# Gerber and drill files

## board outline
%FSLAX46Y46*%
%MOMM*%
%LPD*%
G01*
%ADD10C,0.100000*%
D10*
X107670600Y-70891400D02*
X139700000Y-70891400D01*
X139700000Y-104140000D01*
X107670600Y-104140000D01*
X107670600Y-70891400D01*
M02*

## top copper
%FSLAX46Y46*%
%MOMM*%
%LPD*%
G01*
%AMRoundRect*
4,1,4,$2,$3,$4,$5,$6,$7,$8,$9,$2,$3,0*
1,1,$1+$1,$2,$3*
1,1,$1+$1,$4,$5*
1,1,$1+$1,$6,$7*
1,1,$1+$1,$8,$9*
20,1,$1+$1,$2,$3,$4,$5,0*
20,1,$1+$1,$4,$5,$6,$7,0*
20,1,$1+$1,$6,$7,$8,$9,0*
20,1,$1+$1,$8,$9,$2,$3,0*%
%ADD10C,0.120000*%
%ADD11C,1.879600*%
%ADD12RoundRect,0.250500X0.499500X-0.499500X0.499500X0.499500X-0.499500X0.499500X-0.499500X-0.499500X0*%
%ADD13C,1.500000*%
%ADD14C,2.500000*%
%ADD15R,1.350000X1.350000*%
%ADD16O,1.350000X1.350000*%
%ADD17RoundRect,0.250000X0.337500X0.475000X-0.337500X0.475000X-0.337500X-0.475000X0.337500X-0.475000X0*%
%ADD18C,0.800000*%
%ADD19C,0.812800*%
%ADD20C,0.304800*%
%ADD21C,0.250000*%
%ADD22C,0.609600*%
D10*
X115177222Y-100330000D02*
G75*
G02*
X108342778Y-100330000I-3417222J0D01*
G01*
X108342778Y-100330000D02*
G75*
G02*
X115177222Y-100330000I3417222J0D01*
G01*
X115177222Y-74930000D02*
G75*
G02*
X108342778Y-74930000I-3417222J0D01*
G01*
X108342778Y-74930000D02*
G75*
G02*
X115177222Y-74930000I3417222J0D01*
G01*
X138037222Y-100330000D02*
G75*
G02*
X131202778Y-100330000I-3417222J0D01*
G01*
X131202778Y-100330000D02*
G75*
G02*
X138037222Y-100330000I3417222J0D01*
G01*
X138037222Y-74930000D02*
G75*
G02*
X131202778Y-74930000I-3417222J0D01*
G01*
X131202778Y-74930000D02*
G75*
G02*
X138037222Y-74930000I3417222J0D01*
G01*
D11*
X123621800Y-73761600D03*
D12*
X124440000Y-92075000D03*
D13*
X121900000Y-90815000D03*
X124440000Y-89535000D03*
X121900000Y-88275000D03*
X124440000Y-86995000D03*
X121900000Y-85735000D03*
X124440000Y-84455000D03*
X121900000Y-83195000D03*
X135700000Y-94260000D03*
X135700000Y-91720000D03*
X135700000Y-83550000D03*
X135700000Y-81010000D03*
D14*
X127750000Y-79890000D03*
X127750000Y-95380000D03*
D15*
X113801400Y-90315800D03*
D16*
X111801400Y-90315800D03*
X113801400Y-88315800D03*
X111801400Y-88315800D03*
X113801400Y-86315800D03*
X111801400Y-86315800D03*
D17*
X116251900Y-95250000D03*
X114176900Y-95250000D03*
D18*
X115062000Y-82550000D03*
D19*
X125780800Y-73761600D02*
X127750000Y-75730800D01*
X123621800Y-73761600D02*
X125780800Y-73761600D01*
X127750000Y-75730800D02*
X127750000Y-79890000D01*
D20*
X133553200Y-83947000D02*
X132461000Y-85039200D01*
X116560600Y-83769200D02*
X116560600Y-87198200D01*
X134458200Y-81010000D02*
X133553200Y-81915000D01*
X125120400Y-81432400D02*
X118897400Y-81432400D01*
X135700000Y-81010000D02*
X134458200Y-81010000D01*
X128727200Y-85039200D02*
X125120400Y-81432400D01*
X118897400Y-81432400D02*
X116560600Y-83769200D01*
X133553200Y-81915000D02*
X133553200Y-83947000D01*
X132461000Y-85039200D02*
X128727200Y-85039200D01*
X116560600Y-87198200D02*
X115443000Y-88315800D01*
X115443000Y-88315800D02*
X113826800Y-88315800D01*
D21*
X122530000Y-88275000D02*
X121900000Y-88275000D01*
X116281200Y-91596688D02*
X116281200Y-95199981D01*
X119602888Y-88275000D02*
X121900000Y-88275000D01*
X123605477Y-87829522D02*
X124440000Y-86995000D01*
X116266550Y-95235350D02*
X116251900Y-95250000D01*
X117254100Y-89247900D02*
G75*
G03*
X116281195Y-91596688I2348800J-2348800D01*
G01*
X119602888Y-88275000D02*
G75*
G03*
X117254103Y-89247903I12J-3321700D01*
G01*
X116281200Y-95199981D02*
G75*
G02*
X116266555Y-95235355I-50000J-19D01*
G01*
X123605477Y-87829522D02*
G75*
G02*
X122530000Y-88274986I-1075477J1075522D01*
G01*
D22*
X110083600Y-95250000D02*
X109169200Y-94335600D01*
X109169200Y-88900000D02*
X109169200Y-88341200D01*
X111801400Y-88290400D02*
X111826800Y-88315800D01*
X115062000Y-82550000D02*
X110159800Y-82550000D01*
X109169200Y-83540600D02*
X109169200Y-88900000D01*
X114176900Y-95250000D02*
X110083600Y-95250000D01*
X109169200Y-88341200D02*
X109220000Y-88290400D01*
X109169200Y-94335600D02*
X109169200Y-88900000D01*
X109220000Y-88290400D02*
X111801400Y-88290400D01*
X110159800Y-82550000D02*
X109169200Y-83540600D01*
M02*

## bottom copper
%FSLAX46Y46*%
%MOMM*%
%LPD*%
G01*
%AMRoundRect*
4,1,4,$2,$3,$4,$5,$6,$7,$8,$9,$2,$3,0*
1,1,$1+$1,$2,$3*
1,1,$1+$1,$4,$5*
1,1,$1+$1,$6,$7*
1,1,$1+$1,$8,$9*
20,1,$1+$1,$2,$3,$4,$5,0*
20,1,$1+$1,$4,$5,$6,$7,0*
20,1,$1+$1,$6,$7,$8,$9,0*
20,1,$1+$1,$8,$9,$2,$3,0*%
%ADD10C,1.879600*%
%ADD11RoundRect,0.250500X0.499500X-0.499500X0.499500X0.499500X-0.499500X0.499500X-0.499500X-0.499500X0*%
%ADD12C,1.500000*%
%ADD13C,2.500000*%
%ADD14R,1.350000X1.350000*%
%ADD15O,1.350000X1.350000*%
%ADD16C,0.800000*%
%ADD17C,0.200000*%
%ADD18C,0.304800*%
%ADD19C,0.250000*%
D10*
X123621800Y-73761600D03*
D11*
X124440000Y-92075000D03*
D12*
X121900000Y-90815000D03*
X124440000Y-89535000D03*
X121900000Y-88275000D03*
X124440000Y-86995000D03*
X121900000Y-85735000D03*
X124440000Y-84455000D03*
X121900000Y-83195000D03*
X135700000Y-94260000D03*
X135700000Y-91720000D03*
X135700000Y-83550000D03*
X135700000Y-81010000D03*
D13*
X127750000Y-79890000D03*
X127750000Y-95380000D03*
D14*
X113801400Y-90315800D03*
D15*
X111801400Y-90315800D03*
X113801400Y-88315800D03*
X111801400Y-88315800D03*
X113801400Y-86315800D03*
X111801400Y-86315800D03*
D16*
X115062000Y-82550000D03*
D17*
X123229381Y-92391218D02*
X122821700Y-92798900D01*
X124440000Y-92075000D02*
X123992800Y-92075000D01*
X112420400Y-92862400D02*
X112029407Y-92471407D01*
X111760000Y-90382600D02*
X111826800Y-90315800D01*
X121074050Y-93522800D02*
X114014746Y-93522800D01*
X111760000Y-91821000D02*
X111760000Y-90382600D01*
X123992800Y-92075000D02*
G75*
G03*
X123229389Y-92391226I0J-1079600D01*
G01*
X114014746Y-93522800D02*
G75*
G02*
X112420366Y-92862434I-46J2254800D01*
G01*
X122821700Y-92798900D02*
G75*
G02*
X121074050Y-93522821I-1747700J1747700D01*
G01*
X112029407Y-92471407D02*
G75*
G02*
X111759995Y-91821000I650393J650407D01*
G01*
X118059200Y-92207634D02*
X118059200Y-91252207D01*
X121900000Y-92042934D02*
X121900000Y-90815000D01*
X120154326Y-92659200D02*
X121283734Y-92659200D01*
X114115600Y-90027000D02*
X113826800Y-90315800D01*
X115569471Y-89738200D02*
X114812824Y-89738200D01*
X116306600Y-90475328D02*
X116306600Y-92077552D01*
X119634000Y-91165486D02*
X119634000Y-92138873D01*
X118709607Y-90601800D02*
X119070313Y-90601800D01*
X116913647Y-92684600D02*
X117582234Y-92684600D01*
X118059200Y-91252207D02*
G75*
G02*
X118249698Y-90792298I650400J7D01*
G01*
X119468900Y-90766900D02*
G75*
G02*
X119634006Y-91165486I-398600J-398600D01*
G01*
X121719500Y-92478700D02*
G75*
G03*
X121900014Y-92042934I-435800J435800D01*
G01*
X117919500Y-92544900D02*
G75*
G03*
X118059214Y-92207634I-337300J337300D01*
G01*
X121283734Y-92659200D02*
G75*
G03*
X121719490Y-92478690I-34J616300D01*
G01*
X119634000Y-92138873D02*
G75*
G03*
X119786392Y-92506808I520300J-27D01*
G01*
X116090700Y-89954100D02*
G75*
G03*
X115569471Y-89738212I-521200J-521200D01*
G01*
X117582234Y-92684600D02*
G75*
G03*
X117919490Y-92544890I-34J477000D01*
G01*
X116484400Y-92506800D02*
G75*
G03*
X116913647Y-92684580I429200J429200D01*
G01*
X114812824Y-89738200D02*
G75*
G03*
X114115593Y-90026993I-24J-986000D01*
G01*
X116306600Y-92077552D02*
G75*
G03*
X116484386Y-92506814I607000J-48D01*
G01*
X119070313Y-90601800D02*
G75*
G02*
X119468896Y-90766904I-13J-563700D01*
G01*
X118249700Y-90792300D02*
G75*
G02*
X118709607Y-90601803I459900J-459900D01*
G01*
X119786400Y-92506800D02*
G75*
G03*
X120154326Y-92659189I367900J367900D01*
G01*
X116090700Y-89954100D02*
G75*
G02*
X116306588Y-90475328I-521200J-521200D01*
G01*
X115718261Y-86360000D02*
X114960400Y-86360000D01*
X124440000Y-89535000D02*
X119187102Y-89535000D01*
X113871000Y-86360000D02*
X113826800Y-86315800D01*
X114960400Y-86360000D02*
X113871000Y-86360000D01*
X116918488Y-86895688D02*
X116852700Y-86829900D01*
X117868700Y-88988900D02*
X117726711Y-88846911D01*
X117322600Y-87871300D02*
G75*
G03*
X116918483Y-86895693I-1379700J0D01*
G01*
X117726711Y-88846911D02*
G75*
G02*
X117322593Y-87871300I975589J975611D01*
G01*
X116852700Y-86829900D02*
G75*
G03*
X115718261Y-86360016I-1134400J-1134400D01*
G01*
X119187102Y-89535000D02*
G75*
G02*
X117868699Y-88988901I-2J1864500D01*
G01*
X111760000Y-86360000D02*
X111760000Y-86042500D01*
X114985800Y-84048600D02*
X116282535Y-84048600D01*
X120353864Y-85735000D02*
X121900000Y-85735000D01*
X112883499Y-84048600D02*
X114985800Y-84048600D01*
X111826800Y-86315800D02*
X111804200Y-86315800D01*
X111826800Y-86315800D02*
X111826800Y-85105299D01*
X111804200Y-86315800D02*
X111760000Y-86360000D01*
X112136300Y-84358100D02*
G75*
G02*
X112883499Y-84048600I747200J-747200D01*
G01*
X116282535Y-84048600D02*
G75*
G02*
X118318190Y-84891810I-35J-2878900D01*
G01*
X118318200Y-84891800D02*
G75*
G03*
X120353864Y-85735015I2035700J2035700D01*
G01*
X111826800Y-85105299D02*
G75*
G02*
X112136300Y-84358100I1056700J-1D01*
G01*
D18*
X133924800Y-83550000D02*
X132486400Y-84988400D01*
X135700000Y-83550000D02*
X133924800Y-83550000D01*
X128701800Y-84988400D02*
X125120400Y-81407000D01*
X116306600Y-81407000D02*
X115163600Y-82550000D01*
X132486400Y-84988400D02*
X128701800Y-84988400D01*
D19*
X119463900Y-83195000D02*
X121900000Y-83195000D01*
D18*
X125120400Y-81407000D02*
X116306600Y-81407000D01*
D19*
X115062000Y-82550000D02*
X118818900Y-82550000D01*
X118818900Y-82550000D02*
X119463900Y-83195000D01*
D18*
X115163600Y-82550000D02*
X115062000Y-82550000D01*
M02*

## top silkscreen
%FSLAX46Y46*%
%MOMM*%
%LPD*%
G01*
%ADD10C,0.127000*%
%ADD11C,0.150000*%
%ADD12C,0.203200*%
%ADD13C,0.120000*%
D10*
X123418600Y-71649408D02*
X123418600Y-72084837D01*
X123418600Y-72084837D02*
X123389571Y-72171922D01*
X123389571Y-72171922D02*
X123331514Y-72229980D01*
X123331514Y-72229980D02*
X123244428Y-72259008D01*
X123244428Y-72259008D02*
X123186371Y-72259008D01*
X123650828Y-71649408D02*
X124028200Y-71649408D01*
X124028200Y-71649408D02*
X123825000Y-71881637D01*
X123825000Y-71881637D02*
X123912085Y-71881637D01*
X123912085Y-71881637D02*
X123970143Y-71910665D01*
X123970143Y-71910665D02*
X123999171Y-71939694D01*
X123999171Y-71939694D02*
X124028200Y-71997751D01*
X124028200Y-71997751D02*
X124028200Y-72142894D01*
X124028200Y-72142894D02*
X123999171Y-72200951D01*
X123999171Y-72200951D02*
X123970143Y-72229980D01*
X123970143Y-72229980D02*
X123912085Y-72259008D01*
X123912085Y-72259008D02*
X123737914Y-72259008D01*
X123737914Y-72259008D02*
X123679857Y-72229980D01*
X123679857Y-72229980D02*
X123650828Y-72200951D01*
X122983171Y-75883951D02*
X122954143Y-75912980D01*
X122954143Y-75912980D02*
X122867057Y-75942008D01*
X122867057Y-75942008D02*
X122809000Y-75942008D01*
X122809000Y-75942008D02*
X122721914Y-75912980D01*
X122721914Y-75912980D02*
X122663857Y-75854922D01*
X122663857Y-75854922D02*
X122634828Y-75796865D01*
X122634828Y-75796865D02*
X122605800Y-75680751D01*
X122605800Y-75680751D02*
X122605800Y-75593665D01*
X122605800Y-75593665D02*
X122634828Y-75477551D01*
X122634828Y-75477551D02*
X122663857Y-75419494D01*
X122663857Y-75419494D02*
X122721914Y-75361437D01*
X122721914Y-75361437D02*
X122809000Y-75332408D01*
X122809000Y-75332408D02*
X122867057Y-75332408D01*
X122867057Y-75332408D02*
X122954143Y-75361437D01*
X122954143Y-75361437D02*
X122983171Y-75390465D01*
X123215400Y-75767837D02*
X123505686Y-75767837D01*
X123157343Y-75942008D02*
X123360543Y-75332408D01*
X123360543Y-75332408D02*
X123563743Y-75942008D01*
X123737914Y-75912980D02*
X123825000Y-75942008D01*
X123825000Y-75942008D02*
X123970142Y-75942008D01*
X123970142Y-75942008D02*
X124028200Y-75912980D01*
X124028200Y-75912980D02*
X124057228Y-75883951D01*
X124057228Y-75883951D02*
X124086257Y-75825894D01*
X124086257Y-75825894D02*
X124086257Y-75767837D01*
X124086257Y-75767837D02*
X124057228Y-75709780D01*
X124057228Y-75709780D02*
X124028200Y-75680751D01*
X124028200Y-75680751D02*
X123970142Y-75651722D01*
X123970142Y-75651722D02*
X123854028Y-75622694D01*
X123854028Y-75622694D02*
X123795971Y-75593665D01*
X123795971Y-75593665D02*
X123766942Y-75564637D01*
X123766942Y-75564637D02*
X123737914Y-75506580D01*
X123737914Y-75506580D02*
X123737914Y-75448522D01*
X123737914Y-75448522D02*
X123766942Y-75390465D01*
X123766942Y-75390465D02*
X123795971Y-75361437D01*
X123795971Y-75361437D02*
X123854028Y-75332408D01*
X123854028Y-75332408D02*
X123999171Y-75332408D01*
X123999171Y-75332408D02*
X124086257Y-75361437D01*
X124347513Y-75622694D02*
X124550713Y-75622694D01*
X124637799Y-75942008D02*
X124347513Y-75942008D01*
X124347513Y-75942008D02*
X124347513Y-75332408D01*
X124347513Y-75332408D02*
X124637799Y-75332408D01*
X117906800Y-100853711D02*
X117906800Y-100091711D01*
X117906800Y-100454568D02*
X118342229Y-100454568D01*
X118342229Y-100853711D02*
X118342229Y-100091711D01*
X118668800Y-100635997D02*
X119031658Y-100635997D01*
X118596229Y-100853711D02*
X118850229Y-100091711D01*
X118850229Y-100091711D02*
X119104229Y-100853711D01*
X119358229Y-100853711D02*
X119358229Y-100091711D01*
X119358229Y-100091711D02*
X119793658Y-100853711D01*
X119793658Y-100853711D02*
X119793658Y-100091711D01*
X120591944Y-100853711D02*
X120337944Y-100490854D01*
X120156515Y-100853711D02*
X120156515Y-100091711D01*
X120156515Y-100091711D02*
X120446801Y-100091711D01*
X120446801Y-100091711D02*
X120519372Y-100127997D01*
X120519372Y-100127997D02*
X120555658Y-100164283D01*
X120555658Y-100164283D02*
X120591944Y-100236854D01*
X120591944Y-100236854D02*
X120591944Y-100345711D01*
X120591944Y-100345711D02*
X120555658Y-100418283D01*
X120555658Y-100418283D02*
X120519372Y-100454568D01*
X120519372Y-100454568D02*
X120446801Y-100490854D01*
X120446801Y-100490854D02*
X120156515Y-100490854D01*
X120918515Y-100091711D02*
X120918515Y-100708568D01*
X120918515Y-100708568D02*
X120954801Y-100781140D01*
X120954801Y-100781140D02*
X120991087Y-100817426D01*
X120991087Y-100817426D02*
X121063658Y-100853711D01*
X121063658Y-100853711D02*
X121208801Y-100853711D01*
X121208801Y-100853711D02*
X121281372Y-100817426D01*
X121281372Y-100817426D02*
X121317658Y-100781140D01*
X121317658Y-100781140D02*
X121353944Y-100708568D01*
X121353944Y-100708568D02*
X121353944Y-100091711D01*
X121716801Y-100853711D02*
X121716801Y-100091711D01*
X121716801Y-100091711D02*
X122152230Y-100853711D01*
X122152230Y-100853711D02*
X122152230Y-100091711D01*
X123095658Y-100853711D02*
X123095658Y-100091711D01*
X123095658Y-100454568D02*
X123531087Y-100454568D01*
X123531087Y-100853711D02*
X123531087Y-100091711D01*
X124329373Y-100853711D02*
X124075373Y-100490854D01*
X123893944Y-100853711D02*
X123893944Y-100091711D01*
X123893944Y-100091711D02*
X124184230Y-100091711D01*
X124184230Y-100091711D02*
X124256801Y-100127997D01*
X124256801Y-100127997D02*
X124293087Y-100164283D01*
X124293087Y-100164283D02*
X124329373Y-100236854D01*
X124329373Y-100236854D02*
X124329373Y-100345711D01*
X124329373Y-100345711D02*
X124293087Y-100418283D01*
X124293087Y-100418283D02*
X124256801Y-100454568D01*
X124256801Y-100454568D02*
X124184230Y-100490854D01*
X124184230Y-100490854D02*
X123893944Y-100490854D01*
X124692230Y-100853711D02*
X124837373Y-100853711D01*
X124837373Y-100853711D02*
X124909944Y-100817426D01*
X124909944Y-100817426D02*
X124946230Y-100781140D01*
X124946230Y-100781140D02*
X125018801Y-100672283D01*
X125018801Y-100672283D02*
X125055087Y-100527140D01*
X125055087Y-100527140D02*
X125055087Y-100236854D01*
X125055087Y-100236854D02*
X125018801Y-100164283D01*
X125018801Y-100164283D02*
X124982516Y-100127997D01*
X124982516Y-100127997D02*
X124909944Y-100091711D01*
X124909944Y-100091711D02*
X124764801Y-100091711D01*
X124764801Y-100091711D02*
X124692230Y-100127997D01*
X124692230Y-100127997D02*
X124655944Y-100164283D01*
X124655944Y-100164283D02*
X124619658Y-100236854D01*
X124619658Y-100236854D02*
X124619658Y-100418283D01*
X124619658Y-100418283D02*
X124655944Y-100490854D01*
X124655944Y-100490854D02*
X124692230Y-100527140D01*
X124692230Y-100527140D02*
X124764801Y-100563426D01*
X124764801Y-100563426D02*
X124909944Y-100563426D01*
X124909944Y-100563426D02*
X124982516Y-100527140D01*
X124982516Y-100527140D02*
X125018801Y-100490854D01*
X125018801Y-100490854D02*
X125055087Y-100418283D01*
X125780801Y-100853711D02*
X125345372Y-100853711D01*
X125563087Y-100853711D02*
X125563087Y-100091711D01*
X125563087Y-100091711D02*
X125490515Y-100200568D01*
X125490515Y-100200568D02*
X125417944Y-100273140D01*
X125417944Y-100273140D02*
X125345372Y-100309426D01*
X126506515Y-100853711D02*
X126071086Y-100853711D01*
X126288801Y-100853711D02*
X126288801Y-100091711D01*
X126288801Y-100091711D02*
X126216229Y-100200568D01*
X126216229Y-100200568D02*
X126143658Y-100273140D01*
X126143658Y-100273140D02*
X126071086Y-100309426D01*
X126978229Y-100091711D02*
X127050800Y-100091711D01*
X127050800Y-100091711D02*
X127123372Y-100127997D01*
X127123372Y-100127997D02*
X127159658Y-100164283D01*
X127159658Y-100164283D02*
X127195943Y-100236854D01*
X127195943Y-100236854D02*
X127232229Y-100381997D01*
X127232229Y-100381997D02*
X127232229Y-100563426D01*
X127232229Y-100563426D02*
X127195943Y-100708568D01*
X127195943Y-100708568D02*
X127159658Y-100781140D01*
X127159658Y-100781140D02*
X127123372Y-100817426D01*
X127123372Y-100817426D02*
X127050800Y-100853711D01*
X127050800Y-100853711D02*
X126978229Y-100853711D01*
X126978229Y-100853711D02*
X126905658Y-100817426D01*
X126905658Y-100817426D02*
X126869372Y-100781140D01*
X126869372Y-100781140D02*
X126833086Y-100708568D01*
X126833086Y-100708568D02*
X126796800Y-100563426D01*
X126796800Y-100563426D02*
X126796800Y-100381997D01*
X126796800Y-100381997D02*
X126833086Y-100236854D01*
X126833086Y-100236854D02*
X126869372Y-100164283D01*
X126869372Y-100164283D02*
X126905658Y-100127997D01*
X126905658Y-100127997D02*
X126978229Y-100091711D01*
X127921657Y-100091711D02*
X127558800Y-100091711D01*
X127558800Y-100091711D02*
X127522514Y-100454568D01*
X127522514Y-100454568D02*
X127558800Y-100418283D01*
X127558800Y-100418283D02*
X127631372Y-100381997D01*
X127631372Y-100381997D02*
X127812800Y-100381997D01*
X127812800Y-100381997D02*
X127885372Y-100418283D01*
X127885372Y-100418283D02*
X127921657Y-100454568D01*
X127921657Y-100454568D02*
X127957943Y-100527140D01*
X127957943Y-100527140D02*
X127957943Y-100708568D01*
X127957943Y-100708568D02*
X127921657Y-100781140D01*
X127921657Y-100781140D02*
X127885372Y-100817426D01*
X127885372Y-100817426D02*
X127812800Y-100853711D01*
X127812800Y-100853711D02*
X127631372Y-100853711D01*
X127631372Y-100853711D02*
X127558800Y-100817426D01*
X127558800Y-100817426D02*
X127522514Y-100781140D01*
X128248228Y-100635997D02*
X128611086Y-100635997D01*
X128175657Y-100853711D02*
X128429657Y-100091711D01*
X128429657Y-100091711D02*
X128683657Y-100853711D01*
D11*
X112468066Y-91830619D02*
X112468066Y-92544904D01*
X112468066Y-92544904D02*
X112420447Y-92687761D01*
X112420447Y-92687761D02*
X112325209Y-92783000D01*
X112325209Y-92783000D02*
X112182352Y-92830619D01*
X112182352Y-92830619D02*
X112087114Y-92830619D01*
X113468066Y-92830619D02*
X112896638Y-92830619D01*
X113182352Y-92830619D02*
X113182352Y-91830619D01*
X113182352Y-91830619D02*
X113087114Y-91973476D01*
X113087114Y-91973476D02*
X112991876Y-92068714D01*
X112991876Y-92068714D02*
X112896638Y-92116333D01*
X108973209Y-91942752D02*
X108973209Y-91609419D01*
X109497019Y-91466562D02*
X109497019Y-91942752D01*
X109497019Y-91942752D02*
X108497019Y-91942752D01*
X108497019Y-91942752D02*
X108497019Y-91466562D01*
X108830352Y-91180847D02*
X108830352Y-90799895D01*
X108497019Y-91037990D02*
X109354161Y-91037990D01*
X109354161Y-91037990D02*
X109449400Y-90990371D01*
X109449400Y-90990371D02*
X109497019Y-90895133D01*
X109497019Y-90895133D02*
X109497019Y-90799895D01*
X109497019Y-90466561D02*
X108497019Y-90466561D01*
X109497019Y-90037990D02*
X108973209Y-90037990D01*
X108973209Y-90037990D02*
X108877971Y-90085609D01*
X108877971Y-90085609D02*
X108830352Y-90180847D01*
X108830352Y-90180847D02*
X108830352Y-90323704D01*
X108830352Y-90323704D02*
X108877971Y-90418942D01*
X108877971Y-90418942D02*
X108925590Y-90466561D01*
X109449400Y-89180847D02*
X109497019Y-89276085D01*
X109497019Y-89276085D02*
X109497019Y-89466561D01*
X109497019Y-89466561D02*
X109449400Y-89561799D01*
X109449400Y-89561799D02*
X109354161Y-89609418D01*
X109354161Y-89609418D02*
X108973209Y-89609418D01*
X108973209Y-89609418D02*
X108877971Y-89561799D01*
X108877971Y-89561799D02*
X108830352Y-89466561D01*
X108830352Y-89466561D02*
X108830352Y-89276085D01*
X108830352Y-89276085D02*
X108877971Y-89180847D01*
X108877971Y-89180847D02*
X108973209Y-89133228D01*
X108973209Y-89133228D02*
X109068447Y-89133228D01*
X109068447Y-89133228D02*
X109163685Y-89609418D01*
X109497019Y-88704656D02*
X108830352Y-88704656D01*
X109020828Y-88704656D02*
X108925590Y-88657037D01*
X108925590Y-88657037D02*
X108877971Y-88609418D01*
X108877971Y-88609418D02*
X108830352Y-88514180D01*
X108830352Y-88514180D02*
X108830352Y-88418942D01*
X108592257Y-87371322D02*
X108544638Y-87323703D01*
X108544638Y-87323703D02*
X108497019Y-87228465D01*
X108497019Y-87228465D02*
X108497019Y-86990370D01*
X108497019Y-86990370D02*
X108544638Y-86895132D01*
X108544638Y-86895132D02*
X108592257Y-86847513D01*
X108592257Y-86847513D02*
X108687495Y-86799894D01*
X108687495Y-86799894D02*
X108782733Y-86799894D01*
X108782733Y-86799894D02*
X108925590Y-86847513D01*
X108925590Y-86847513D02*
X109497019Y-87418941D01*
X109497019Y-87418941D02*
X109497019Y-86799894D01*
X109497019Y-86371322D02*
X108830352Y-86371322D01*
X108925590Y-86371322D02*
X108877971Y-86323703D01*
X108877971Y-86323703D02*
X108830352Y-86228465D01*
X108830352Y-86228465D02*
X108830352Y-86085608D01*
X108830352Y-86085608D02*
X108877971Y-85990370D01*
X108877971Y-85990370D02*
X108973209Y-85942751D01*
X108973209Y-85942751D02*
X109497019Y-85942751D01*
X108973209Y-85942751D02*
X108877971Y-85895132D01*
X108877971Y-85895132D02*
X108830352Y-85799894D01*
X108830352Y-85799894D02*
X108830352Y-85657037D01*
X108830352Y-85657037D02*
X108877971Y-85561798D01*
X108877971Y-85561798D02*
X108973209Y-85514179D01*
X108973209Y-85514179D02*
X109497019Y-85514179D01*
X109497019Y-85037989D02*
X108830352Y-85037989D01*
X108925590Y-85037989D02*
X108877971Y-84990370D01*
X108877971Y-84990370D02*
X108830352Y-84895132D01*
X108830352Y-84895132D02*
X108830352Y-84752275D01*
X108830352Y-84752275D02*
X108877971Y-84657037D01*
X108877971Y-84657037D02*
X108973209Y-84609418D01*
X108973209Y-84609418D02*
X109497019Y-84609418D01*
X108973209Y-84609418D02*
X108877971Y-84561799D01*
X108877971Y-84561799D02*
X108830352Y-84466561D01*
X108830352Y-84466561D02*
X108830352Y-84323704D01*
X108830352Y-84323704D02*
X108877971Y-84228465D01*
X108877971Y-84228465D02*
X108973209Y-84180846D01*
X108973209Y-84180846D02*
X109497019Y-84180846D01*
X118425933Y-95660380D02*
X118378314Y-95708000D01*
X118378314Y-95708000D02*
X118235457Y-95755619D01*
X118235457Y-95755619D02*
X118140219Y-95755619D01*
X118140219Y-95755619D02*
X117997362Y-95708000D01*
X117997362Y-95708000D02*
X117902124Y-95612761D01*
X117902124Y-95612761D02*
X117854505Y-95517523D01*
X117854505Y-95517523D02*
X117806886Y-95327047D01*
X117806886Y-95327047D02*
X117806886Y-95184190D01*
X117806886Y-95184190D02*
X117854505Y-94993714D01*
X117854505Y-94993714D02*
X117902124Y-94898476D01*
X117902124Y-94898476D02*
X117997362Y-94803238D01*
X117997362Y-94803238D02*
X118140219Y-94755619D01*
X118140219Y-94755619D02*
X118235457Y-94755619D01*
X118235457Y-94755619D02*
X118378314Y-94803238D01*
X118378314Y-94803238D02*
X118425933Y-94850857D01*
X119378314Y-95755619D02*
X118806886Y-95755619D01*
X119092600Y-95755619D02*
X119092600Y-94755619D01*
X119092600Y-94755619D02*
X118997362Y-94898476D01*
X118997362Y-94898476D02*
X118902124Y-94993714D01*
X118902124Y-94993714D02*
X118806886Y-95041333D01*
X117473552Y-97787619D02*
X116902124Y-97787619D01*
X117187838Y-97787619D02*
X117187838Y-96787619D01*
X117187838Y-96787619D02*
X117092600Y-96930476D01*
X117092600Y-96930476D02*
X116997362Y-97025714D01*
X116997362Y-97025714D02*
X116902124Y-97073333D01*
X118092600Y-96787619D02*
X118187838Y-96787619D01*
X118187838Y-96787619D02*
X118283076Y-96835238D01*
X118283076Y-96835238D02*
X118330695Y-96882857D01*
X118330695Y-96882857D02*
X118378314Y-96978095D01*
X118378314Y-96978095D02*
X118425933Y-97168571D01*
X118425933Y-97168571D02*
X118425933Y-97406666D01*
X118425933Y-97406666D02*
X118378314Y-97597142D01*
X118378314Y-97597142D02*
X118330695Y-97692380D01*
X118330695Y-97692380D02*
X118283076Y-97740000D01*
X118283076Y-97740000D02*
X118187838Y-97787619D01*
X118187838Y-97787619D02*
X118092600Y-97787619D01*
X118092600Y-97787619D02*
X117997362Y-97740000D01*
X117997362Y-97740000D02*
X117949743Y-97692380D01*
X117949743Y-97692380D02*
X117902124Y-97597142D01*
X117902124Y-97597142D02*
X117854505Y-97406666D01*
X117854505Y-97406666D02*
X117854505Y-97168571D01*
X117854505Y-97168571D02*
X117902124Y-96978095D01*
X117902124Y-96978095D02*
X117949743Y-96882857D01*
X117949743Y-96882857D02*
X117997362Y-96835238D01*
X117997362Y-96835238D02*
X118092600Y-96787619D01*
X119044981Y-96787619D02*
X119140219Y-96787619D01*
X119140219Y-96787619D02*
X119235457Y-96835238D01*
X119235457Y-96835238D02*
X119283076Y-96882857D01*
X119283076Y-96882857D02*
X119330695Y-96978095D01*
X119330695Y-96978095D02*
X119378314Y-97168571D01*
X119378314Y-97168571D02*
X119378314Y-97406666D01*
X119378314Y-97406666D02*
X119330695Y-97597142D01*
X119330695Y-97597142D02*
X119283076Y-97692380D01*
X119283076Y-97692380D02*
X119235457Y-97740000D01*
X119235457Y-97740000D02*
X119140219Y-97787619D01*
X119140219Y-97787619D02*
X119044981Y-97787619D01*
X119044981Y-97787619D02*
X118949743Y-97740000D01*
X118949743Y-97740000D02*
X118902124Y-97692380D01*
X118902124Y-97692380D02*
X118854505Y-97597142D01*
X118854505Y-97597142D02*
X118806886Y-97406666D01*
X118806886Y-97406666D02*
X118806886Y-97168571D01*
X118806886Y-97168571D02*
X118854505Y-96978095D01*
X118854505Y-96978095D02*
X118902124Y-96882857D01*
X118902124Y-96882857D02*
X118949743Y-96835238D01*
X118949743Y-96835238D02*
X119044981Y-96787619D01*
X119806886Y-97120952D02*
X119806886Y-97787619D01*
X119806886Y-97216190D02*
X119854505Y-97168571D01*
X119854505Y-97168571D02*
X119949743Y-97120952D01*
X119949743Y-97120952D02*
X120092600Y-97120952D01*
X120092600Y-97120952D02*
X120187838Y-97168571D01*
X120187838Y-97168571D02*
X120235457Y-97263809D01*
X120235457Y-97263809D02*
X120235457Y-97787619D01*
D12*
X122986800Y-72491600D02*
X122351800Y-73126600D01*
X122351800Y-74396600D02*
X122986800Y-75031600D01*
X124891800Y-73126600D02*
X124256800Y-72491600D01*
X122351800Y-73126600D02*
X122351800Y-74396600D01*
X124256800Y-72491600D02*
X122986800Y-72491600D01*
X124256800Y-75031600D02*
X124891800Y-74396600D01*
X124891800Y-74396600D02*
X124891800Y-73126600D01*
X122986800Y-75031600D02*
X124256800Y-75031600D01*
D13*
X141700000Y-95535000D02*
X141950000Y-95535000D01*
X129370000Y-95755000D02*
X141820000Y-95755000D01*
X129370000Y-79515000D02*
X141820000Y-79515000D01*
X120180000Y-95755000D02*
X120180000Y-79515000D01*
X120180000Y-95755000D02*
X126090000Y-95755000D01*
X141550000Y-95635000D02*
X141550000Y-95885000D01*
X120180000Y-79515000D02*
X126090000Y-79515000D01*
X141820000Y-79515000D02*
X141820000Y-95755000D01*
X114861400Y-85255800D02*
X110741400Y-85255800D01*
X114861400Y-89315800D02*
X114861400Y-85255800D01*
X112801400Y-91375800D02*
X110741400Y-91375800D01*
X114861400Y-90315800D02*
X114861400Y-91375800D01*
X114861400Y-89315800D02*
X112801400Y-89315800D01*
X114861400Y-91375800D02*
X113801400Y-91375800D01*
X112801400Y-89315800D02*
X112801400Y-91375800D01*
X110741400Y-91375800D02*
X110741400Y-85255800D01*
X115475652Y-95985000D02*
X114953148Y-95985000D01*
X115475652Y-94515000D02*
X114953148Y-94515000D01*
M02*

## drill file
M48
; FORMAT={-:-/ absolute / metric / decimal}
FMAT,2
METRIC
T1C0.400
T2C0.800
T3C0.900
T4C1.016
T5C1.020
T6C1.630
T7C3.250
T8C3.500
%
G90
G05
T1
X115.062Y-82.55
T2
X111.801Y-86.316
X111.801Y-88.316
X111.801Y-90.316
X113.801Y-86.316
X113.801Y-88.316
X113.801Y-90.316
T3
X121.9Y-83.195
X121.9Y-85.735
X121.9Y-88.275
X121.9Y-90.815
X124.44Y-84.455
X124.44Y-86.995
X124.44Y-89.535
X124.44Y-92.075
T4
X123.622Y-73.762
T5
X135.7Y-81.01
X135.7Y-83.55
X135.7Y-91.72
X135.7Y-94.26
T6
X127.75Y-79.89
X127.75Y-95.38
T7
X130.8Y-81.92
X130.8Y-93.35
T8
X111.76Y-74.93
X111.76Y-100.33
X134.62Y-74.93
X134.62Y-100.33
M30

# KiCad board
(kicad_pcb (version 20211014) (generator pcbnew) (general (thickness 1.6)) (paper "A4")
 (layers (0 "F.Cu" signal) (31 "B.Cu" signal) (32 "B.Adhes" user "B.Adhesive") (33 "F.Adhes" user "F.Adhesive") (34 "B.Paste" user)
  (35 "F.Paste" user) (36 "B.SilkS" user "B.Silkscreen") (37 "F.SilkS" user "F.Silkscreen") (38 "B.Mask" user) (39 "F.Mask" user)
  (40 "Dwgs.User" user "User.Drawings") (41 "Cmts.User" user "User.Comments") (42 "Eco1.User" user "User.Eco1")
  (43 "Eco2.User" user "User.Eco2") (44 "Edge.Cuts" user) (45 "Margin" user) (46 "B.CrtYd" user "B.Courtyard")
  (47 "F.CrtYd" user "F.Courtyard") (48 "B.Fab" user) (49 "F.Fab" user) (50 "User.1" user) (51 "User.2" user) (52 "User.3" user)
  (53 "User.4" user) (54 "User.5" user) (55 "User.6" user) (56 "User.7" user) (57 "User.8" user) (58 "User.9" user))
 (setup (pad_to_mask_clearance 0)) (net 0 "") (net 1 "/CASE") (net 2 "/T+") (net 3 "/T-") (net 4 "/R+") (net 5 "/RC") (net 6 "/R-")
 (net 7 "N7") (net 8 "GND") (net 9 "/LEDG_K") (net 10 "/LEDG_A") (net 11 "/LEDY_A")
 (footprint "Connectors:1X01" (layer "F.Cu") (at 123.6218 73.7616)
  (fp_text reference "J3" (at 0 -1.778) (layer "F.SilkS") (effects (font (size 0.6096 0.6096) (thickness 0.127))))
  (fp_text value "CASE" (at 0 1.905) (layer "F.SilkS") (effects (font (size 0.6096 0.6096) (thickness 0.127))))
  (fp_line (start -0.635 -1.27) (end -1.27 -0.635) (layer "F.SilkS") (width 0.2032))
  (fp_line (start -1.27 0.635) (end -0.635 1.27) (layer "F.SilkS") (width 0.2032))
  (fp_line (start 1.27 -0.635) (end 0.635 -1.27) (layer "F.SilkS") (width 0.2032))
  (fp_line (start -1.27 -0.635) (end -1.27 0.635) (layer "F.SilkS") (width 0.2032))
  (fp_line (start 0.635 -1.27) (end -0.635 -1.27) (layer "F.SilkS") (width 0.2032))
  (fp_line (start 0.635 1.27) (end 1.27 0.635) (layer "F.SilkS") (width 0.2032))
  (fp_line (start 1.27 0.635) (end 1.27 -0.635) (layer "F.SilkS") (width 0.2032))
  (fp_line (start -0.635 1.27) (end 0.635 1.27) (layer "F.SilkS") (width 0.2032))
  (pad "1" thru_hole circle locked (at 0 0) (size 1.8796 1.8796) (drill 1.016) (layers *.Cu *.Mask) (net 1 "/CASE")
   (solder_mask_margin 0.1016)))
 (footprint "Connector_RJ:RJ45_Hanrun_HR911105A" (layer "F.Cu") (at 124.44 92.075 90)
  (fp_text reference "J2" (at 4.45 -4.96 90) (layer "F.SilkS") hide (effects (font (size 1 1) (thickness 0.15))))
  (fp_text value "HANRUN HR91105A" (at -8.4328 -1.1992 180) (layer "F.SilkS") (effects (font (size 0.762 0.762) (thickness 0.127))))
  (fp_line (start -3.46 17.26) (end -3.46 17.51) (layer "F.SilkS") (width 0.12))
  (fp_line (start -3.68 4.93) (end -3.68 17.38) (layer "F.SilkS") (width 0.12))
  (fp_line (start 12.56 4.93) (end 12.56 17.38) (layer "F.SilkS") (width 0.12))
  (fp_line (start -3.68 -4.26) (end 12.56 -4.26) (layer "F.SilkS") (width 0.12))
  (fp_line (start -3.68 -4.26) (end -3.68 1.65) (layer "F.SilkS") (width 0.12))
  (fp_line (start -3.56 17.11) (end -3.81 17.11) (layer "F.SilkS") (width 0.12))
  (fp_line (start 12.56 -4.26) (end 12.56 1.65) (layer "F.SilkS") (width 0.12))
  (fp_line (start 12.56 17.38) (end -3.68 17.38) (layer "F.SilkS") (width 0.12))
  (pad "" np_thru_hole circle (at 10.155 6.36 90) (size 3.25 3.25) (drill 3.25) (layers *.Cu *.Mask))
  (pad "" np_thru_hole circle (at -1.275 6.36 90) (size 3.25 3.25) (drill 3.25) (layers *.Cu *.Mask))
  (pad "1" thru_hole roundrect (at 0 0 90) (size 1.5 1.5) (drill 0.9) (layers *.Cu *.Mask) (roundrect_rratio 0.167) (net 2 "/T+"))
  (pad "2" thru_hole circle (at 1.26 -2.54 90) (size 1.5 1.5) (drill 0.9) (layers *.Cu *.Mask) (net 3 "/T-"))
  (pad "3" thru_hole circle (at 2.54 0 90) (size 1.5 1.5) (drill 0.9) (layers *.Cu *.Mask) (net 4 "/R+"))
  (pad "4" thru_hole circle (at 3.8 -2.54 90) (size 1.5 1.5) (drill 0.9) (layers *.Cu *.Mask) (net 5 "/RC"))
  (pad "5" thru_hole circle (at 5.08 0 90) (size 1.5 1.5) (drill 0.9) (layers *.Cu *.Mask) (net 5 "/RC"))
  (pad "6" thru_hole circle (at 6.34 -2.54 180) (size 1.5 1.5) (drill 0.9) (layers *.Cu *.Mask) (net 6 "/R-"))
  (pad "7" thru_hole circle (at 7.62 0 90) (size 1.5 1.5) (drill 0.9) (layers *.Cu *.Mask) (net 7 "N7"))
  (pad "8" thru_hole circle (at 8.88 -2.54 90) (size 1.5 1.5) (drill 0.9) (layers *.Cu *.Mask) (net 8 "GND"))
  (pad "9" thru_hole circle (at -2.185 11.26 90) (size 1.5 1.5) (drill 1.02) (layers *.Cu *.Mask) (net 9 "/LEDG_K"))
  (pad "10" thru_hole circle (at 0.355 11.26 90) (size 1.5 1.5) (drill 1.02) (layers *.Cu *.Mask) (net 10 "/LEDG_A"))
  (pad "11" thru_hole circle (at 8.525 11.26 90) (size 1.5 1.5) (drill 1.02) (layers *.Cu *.Mask) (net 8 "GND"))
  (pad "12" thru_hole circle (at 11.065 11.26 90) (size 1.5 1.5) (drill 1.02) (layers *.Cu *.Mask) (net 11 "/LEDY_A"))
  (pad "SH" thru_hole circle (at 12.185 3.31 90) (size 2.5 2.5) (drill 1.63) (layers *.Cu *.Mask) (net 1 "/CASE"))
  (pad "SH" thru_hole circle (at -3.305 3.31 90) (size 2.5 2.5) (drill 1.63) (layers *.Cu *.Mask) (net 1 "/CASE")))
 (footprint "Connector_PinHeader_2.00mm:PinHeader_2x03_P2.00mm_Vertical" (layer "F.Cu") (at 113.8014 90.3158 180)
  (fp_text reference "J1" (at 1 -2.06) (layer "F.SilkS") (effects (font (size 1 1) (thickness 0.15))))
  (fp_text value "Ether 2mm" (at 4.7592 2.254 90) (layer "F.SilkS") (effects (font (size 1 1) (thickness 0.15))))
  (fp_line (start -1.06 5.06) (end 3.06 5.06) (layer "F.SilkS") (width 0.12))
  (fp_line (start -1.06 1) (end -1.06 5.06) (layer "F.SilkS") (width 0.12))
  (fp_line (start 1 -1.06) (end 3.06 -1.06) (layer "F.SilkS") (width 0.12))
  (fp_line (start -1.06 0) (end -1.06 -1.06) (layer "F.SilkS") (width 0.12))
  (fp_line (start -1.06 1) (end 1 1) (layer "F.SilkS") (width 0.12))
  (fp_line (start -1.06 -1.06) (end 0 -1.06) (layer "F.SilkS") (width 0.12))
  (fp_line (start 1 1) (end 1 -1.06) (layer "F.SilkS") (width 0.12))
  (fp_line (start 3.06 -1.06) (end 3.06 5.06) (layer "F.SilkS") (width 0.12))
  (pad "1" thru_hole rect (at 0 0 180) (size 1.35 1.35) (drill 0.8) (layers *.Cu *.Mask) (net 3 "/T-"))
  (pad "2" thru_hole oval (at 2 0 180) (size 1.35 1.35) (drill 0.8) (layers *.Cu *.Mask) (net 2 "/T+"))
  (pad "3" thru_hole oval (at 0 2 180) (size 1.35 1.35) (drill 0.8) (layers *.Cu *.Mask) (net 11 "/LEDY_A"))
  (pad "4" thru_hole oval (at 2 2 180) (size 1.35 1.35) (drill 0.8) (layers *.Cu *.Mask) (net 8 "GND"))
  (pad "5" thru_hole oval (at 0 4 180) (size 1.35 1.35) (drill 0.8) (layers *.Cu *.Mask) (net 4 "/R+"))
  (pad "6" thru_hole oval (at 2 4 180) (size 1.35 1.35) (drill 0.8) (layers *.Cu *.Mask) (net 6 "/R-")))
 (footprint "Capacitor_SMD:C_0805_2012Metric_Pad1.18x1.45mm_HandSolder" (layer "F.Cu") (at 115.2144 95.25 180)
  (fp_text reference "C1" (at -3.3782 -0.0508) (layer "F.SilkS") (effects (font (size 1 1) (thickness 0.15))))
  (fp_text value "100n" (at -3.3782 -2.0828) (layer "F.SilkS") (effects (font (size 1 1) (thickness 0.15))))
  (fp_line (start -0.261252 -0.735) (end 0.261252 -0.735) (layer "F.SilkS") (width 0.12))
  (fp_line (start -0.261252 0.735) (end 0.261252 0.735) (layer "F.SilkS") (width 0.12))
  (pad "1" smd roundrect (at -1.0375 0 180) (size 1.175 1.45) (layers "F.Cu" "F.Paste" "F.Mask") (roundrect_rratio 0.2127659574)
   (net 5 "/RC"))
  (pad "2" smd roundrect (at 1.0375 0 180) (size 1.175 1.45) (layers "F.Cu" "F.Paste" "F.Mask") (roundrect_rratio 0.2127659574)
   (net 8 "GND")))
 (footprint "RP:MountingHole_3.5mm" (layer "F.Cu") (at 111.76 100.33)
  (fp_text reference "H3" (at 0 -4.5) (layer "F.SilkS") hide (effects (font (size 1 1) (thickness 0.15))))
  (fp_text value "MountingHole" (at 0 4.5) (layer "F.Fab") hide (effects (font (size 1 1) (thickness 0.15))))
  (fp_circle (center 0 0) (end 3.417222 0) (layer "F.Cu") (width 0.12) (fill none))
  (pad "" np_thru_hole circle (at 0 0) (size 3.500001 3.500001) (drill 3.500001) (layers *.Mask)))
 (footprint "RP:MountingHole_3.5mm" (layer "F.Cu") (at 111.76 74.93)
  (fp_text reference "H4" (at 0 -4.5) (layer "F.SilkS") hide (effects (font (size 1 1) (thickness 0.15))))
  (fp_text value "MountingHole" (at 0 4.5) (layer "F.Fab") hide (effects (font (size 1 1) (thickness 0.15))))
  (fp_circle (center 0 0) (end 3.417222 0) (layer "F.Cu") (width 0.12) (fill none))
  (pad "" np_thru_hole circle (at 0 0) (size 3.500001 3.500001) (drill 3.500001) (layers *.Mask)))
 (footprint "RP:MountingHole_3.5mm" (layer "F.Cu") (at 134.62 100.33)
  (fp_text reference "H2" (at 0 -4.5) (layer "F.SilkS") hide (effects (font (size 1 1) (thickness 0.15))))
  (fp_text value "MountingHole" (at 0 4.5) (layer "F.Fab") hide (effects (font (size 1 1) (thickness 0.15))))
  (fp_circle (center 0 0) (end 3.417222 0) (layer "F.Cu") (width 0.12) (fill none))
  (pad "" np_thru_hole circle (at 0 0) (size 3.500001 3.500001) (drill 3.500001) (layers *.Mask)))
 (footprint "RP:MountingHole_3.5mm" (layer "F.Cu") (at 134.62 74.93)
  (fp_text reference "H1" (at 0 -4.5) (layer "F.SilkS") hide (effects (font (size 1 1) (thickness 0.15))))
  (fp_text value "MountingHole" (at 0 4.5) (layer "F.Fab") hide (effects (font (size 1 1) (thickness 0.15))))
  (fp_circle (center 0 0) (end 3.417222 0) (layer "F.Cu") (width 0.12) (fill none))
  (pad "" np_thru_hole circle (at 0 0) (size 3.500001 3.500001) (drill 3.500001) (layers *.Mask)))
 (gr_rect locked (start 107.6706 70.8914) (end 139.7 104.14) (layer "Edge.Cuts") (width 0.1) (fill none))
 (segment (start 125.7808 73.7616) (end 127.75 75.7308) (width 0.8128) (layer "F.Cu") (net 1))
 (segment (start 123.6218 73.7616) (end 125.7808 73.7616) (width 0.8128) (layer "F.Cu") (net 1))
 (segment (start 127.75 75.7308) (end 127.75 79.89) (width 0.8128) (layer "F.Cu") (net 1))
 (segment (start 133.5532 83.947) (end 132.461 85.0392) (width 0.3048) (layer "F.Cu") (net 11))
 (segment (start 116.5606 83.7692) (end 116.5606 87.1982) (width 0.3048) (layer "F.Cu") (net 11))
 (segment (start 134.4582 81.01) (end 133.5532 81.915) (width 0.3048) (layer "F.Cu") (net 11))
 (segment (start 125.1204 81.4324) (end 118.8974 81.4324) (width 0.3048) (layer "F.Cu") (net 11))
 (segment (start 135.7 81.01) (end 134.4582 81.01) (width 0.3048) (layer "F.Cu") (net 11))
 (segment (start 128.7272 85.0392) (end 125.1204 81.4324) (width 0.3048) (layer "F.Cu") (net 11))
 (segment (start 118.8974 81.4324) (end 116.5606 83.7692) (width 0.3048) (layer "F.Cu") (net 11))
 (segment (start 133.5532 81.915) (end 133.5532 83.947) (width 0.3048) (layer "F.Cu") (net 11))
 (segment (start 132.461 85.0392) (end 128.7272 85.0392) (width 0.3048) (layer "F.Cu") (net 11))
 (segment (start 116.5606 87.1982) (end 115.443 88.3158) (width 0.3048) (layer "F.Cu") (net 11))
 (segment (start 115.443 88.3158) (end 113.8268 88.3158) (width 0.3048) (layer "F.Cu") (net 11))
 (segment (start 123.229381 92.391218) (end 122.8217 92.7989) (width 0.2) (layer "B.Cu") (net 2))
 (segment (start 124.44 92.075) (end 123.9928 92.075) (width 0.2) (layer "B.Cu") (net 2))
 (segment (start 112.4204 92.8624) (end 112.029407 92.471407) (width 0.2) (layer "B.Cu") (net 2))
 (segment (start 111.76 90.3826) (end 111.8268 90.3158) (width 0.2) (layer "B.Cu") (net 2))
 (segment (start 121.07405 93.5228) (end 114.014746 93.5228) (width 0.2) (layer "B.Cu") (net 2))
 (segment (start 111.76 91.821) (end 111.76 90.3826) (width 0.2) (layer "B.Cu") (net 2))
 (arc (start 123.9928 92.075) (mid 123.57964 92.157182) (end 123.229381 92.391218) (width 0.2) (layer "B.Cu") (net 2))
 (arc (start 114.014746 93.5228) (mid 113.151892 93.351167) (end 112.4204 92.8624) (width 0.2) (layer "B.Cu") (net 2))
 (arc (start 122.8217 92.7989) (mid 122.019871 93.334664) (end 121.07405 93.5228) (width 0.2) (layer "B.Cu") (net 2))
 (arc (start 112.029407 92.471407) (mid 111.830016 92.172997) (end 111.76 91.821) (width 0.2) (layer "B.Cu") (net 2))
 (segment (start 118.0592 92.207634) (end 118.0592 91.252207) (width 0.2) (layer "B.Cu") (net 3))
 (segment (start 121.9 92.042934) (end 121.9 90.815) (width 0.2) (layer "B.Cu") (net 3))
 (segment (start 120.154326 92.6592) (end 121.283734 92.6592) (width 0.2) (layer "B.Cu") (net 3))
 (segment (start 114.1156 90.027) (end 113.8268 90.3158) (width 0.2) (layer "B.Cu") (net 3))
 (segment (start 115.569471 89.7382) (end 114.812824 89.7382) (width 0.2) (layer "B.Cu") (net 3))
 (segment (start 116.3066 90.475328) (end 116.3066 92.077552) (width 0.2) (layer "B.Cu") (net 3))
 (segment (start 119.634 91.165486) (end 119.634 92.138873) (width 0.2) (layer "B.Cu") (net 3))
 (segment (start 118.709607 90.6018) (end 119.070313 90.6018) (width 0.2) (layer "B.Cu") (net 3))
 (segment (start 116.913647 92.6846) (end 117.582234 92.6846) (width 0.2) (layer "B.Cu") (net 3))
 (arc (start 118.0592 91.252207) (mid 118.108709 91.003307) (end 118.2497 90.7923) (width 0.2) (layer "B.Cu") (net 3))
 (arc (start 119.4689 90.7669) (mid 119.591091 90.949772) (end 119.634 91.165486) (width 0.2) (layer "B.Cu") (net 3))
 (arc (start 121.7195 92.4787) (mid 121.853089 92.278768) (end 121.9 92.042934) (width 0.2) (layer "B.Cu") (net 3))
 (arc (start 117.9195 92.5449) (mid 118.022893 92.390161) (end 118.0592 92.207634) (width 0.2) (layer "B.Cu") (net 3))
 (arc (start 121.283734 92.6592) (mid 121.519568 92.612289) (end 121.7195 92.4787) (width 0.2) (layer "B.Cu") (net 3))
 (arc (start 119.634 92.138873) (mid 119.673607 92.337993) (end 119.7864 92.5068) (width 0.2) (layer "B.Cu") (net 3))
 (arc (start 116.0907 89.9541) (mid 115.851558 89.79431) (end 115.569471 89.7382) (width 0.2) (layer "B.Cu") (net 3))
 (arc (start 117.582234 92.6846) (mid 117.764761 92.648293) (end 117.9195 92.5449) (width 0.2) (layer "B.Cu") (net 3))
 (arc (start 116.4844 92.5068) (mid 116.68134 92.638391) (end 116.913647 92.6846) (width 0.2) (layer "B.Cu") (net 3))
 (arc (start 114.812824 89.7382) (mid 114.435489 89.813256) (end 114.1156 90.027) (width 0.2) (layer "B.Cu") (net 3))
 (arc (start 116.3066 92.077552) (mid 116.352808 92.309859) (end 116.4844 92.5068) (width 0.2) (layer "B.Cu") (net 3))
 (arc (start 119.070313 90.6018) (mid 119.286026 90.644708) (end 119.4689 90.7669) (width 0.2) (layer "B.Cu") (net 3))
 (arc (start 118.2497 90.7923) (mid 118.460707 90.651309) (end 118.709607 90.6018) (width 0.2) (layer "B.Cu") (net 3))
 (arc (start 119.7864 92.5068) (mid 119.955205 92.619592) (end 120.154326 92.6592) (width 0.2) (layer "B.Cu") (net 3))
 (arc (start 116.0907 89.9541) (mid 116.250489 90.193241) (end 116.3066 90.475328) (width 0.2) (layer "B.Cu") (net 3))
 (segment (start 115.718261 86.36) (end 114.9604 86.36) (width 0.2) (layer "B.Cu") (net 4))
 (segment (start 124.44 89.535) (end 119.187102 89.535) (width 0.2) (layer "B.Cu") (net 4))
 (segment (start 113.871 86.36) (end 113.8268 86.3158) (width 0.2) (layer "B.Cu") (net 4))
 (segment (start 114.9604 86.36) (end 113.871 86.36) (width 0.2) (layer "B.Cu") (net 4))
 (segment (start 116.918488 86.895688) (end 116.8527 86.8299) (width 0.2) (layer "B.Cu") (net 4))
 (segment (start 117.8687 88.9889) (end 117.726711 88.846911) (width 0.2) (layer "B.Cu") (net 4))
 (arc (start 117.3226 87.8713) (mid 117.217574 87.343302) (end 116.918488 86.895688) (width 0.2) (layer "B.Cu") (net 4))
 (arc (start 117.726711 88.846911) (mid 117.427625 88.399297) (end 117.3226 87.8713) (width 0.2) (layer "B.Cu") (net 4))
 (arc (start 116.8527 86.8299) (mid 116.332214 86.482123) (end 115.718261 86.36) (width 0.2) (layer "B.Cu") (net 4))
 (arc (start 119.187102 89.535) (mid 118.473587 89.393073) (end 117.8687 88.9889) (width 0.2) (layer "B.Cu") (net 4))
 (segment (start 122.53 88.275) (end 121.9 88.275) (width 0.25) (layer "F.Cu") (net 5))
 (segment (start 116.2812 91.596688) (end 116.2812 95.199981) (width 0.25) (layer "F.Cu") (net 5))
 (segment (start 119.602888 88.275) (end 121.9 88.275) (width 0.25) (layer "F.Cu") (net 5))
 (segment (start 123.605477 87.829522) (end 124.44 86.995) (width 0.25) (layer "F.Cu") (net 5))
 (segment (start 116.26655 95.23535) (end 116.2519 95.25) (width 0.25) (layer "F.Cu") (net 5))
 (arc (start 117.2541 89.2479) (mid 116.534048 90.325533) (end 116.2812 91.596688) (width 0.25) (layer "F.Cu") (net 5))
 (arc (start 119.602888 88.275) (mid 118.331733 88.527848) (end 117.2541 89.2479) (width 0.25) (layer "F.Cu") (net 5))
 (arc (start 116.2812 95.199981) (mid 116.277392 95.219122) (end 116.26655 95.23535) (width 0.25) (layer "F.Cu") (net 5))
 (arc (start 123.605477 87.829522) (mid 123.112044 88.159224) (end 122.53 88.275) (width 0.25) (layer "F.Cu") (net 5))
 (segment (start 111.76 86.36) (end 111.76 86.0425) (width 0.2) (layer "B.Cu") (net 6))
 (segment (start 114.9858 84.0486) (end 116.282535 84.0486) (width 0.2) (layer "B.Cu") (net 6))
 (segment (start 120.353864 85.735) (end 121.9 85.735) (width 0.2) (layer "B.Cu") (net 6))
 (segment (start 112.883499 84.0486) (end 114.9858 84.0486) (width 0.2) (layer "B.Cu") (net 6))
 (segment (start 111.8268 86.3158) (end 111.8042 86.3158) (width 0.2) (layer "B.Cu") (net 6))
 (segment (start 111.8268 86.3158) (end 111.8268 85.105299) (width 0.2) (layer "B.Cu") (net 6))
 (segment (start 111.8042 86.3158) (end 111.76 86.36) (width 0.2) (layer "B.Cu") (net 6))
 (arc (start 112.1363 84.3581) (mid 112.479117 84.129036) (end 112.883499 84.0486) (width 0.2) (layer "B.Cu") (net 6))
 (arc (start 116.282535 84.0486) (mid 117.384228 84.26774) (end 118.3182 84.8918) (width 0.2) (layer "B.Cu") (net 6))
 (arc (start 118.3182 84.8918) (mid 119.25217 85.515859) (end 120.353864 85.735) (width 0.2) (layer "B.Cu") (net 6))
 (arc (start 111.8268 85.105299) (mid 111.907236 84.700917) (end 112.1363 84.3581) (width 0.2) (layer "B.Cu") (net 6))
 (segment (start 110.0836 95.25) (end 109.1692 94.3356) (width 0.6096) (layer "F.Cu") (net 8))
 (segment (start 109.1692 88.9) (end 109.1692 88.3412) (width 0.6096) (layer "F.Cu") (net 8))
 (segment (start 111.8014 88.2904) (end 111.8268 88.3158) (width 0.6096) (layer "F.Cu") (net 8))
 (segment (start 115.062 82.55) (end 110.1598 82.55) (width 0.6096) (layer "F.Cu") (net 8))
 (segment (start 109.1692 83.5406) (end 109.1692 88.9) (width 0.6096) (layer "F.Cu") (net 8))
 (segment (start 114.1769 95.25) (end 110.0836 95.25) (width 0.6096) (layer "F.Cu") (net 8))
 (segment (start 109.1692 88.3412) (end 109.22 88.2904) (width 0.6096) (layer "F.Cu") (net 8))
 (segment (start 109.1692 94.3356) (end 109.1692 88.9) (width 0.6096) (layer "F.Cu") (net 8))
 (segment (start 109.22 88.2904) (end 111.8014 88.2904) (width 0.6096) (layer "F.Cu") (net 8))
 (segment (start 110.1598 82.55) (end 109.1692 83.5406) (width 0.6096) (layer "F.Cu") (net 8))
 (via (at 115.062 82.55) (size 0.8) (drill 0.4) (layers "F.Cu" "B.Cu") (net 8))
 (segment (start 133.9248 83.55) (end 132.4864 84.9884) (width 0.3048) (layer "B.Cu") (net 8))
 (segment (start 135.7 83.55) (end 133.9248 83.55) (width 0.3048) (layer "B.Cu") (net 8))
 (segment (start 128.7018 84.9884) (end 125.1204 81.407) (width 0.3048) (layer "B.Cu") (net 8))
 (segment (start 116.3066 81.407) (end 115.1636 82.55) (width 0.3048) (layer "B.Cu") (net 8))
 (segment (start 132.4864 84.9884) (end 128.7018 84.9884) (width 0.3048) (layer "B.Cu") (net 8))
 (segment (start 119.4639 83.195) (end 121.9 83.195) (width 0.25) (layer "B.Cu") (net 8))
 (segment (start 125.1204 81.407) (end 116.3066 81.407) (width 0.3048) (layer "B.Cu") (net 8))
 (segment (start 115.062 82.55) (end 118.8189 82.55) (width 0.25) (layer "B.Cu") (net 8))
 (segment (start 118.8189 82.55) (end 119.4639 83.195) (width 0.25) (layer "B.Cu") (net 8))
 (segment (start 115.1636 82.55) (end 115.062 82.55) (width 0.3048) (layer "B.Cu") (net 8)))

